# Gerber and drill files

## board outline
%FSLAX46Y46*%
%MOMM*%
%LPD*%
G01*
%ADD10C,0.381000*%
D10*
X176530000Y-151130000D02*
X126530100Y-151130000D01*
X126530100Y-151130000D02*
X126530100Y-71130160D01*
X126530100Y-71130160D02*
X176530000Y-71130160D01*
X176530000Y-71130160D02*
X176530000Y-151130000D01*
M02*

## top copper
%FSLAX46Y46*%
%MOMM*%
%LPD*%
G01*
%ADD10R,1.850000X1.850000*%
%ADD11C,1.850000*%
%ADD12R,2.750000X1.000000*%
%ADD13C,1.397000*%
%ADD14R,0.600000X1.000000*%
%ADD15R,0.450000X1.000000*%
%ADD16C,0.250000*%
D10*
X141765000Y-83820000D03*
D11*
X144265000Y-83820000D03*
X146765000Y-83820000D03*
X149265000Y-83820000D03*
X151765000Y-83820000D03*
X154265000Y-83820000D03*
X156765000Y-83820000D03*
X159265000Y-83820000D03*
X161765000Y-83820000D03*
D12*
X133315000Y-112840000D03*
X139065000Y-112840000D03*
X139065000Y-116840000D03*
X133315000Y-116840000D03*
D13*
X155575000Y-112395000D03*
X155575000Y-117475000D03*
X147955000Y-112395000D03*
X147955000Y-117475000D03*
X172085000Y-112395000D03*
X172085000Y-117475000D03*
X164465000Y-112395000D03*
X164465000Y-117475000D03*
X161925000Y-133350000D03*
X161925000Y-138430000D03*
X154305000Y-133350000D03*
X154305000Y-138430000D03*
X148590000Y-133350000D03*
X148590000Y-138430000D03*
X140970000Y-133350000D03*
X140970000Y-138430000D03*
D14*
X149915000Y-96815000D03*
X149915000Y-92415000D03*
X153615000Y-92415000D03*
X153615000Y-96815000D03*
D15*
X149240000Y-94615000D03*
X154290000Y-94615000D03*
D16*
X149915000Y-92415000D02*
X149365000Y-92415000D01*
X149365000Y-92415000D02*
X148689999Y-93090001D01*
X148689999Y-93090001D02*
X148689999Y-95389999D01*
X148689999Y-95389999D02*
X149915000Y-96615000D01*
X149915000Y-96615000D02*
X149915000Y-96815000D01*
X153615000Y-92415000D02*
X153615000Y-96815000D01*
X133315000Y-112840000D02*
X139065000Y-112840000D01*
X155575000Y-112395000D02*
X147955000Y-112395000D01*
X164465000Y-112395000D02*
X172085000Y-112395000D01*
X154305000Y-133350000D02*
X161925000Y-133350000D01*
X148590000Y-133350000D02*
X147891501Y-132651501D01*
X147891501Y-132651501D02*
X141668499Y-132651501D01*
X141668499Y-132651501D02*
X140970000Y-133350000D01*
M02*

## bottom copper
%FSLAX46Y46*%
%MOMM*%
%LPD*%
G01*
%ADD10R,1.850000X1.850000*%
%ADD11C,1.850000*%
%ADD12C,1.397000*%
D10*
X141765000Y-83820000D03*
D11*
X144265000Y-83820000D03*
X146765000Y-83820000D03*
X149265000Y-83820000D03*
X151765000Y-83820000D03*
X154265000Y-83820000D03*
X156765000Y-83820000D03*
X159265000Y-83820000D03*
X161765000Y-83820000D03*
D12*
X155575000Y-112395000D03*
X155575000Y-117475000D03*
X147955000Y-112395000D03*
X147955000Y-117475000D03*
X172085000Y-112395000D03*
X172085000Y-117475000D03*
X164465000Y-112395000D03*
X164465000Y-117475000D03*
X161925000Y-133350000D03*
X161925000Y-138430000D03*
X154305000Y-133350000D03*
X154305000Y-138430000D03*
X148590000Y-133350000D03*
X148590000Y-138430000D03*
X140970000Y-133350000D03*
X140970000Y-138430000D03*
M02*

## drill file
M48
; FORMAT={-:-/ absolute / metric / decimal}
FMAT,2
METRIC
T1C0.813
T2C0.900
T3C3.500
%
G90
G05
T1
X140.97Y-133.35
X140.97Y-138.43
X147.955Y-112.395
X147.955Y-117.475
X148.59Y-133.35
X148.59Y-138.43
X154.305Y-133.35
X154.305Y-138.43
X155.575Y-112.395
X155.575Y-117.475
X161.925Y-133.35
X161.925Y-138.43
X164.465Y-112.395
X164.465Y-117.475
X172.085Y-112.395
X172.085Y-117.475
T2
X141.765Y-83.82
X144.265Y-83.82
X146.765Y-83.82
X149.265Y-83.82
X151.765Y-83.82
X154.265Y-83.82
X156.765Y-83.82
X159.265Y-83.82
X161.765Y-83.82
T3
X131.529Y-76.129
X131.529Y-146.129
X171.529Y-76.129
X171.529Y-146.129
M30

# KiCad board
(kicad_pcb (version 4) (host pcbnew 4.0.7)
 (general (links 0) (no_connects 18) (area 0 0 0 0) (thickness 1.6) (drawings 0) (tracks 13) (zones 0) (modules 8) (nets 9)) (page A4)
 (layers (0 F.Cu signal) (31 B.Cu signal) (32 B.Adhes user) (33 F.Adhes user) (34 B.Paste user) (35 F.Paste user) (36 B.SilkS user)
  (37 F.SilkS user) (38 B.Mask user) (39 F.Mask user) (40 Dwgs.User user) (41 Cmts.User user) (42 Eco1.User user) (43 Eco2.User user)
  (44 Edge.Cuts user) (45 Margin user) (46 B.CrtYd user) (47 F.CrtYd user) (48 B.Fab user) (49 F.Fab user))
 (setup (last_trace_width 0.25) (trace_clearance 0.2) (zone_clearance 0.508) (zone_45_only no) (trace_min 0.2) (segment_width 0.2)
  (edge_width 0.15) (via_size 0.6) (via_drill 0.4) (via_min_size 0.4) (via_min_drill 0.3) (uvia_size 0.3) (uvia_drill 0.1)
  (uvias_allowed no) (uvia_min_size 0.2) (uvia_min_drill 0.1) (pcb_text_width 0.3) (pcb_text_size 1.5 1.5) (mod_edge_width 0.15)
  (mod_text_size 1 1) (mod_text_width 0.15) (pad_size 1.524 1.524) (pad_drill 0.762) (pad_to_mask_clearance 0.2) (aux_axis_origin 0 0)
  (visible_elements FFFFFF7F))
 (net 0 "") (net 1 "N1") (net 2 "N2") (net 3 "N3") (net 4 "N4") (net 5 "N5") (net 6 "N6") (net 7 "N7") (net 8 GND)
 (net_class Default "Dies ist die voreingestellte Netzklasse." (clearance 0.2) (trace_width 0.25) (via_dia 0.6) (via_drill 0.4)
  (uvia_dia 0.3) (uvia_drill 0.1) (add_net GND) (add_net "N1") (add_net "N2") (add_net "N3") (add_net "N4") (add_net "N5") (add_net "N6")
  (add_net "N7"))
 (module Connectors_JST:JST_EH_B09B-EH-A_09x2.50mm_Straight (layer B.Cu) (at 141.765 83.82)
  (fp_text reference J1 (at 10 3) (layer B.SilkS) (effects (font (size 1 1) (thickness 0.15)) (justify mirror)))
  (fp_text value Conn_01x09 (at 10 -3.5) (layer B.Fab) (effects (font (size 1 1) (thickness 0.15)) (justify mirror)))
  (pad 1 thru_hole rect (at 0 0) (size 1.85 1.85) (drill 0.9) (layers *.Cu *.Mask) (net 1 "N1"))
  (pad 2 thru_hole circle (at 2.5 0) (size 1.85 1.85) (drill 0.9) (layers *.Cu *.Mask) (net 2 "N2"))
  (pad 3 thru_hole circle (at 5 0) (size 1.85 1.85) (drill 0.9) (layers *.Cu *.Mask))
  (pad 4 thru_hole circle (at 7.5 0) (size 1.85 1.85) (drill 0.9) (layers *.Cu *.Mask) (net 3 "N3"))
  (pad 5 thru_hole circle (at 10 0) (size 1.85 1.85) (drill 0.9) (layers *.Cu *.Mask) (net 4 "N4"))
  (pad 6 thru_hole circle (at 12.5 0) (size 1.85 1.85) (drill 0.9) (layers *.Cu *.Mask) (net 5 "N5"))
  (pad 7 thru_hole circle (at 15 0) (size 1.85 1.85) (drill 0.9) (layers *.Cu *.Mask) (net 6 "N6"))
  (pad 8 thru_hole circle (at 17.5 0) (size 1.85 1.85) (drill 0.9) (layers *.Cu *.Mask) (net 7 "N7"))
  (pad 9 thru_hole circle (at 20 0) (size 1.85 1.85) (drill 0.9) (layers *.Cu *.Mask) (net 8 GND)))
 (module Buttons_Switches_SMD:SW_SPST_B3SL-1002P (layer F.Cu) (at 136.19 114.84)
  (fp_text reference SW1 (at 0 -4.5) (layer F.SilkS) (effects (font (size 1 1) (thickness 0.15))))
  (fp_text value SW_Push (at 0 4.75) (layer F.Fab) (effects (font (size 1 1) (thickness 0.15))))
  (pad 1 smd rect (at -2.875 -2) (size 2.75 1) (layers F.Cu F.Paste F.Mask) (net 3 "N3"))
  (pad 1 smd rect (at 2.875 -2) (size 2.75 1) (layers F.Cu F.Paste F.Mask) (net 3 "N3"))
  (pad 2 smd rect (at 2.875 2) (size 2.75 1) (layers F.Cu F.Paste F.Mask) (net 8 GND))
  (pad 2 smd rect (at -2.875 2) (size 2.75 1) (layers F.Cu F.Paste F.Mask) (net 8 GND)))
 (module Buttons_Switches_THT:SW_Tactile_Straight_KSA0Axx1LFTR (layer F.Cu) (at 147.955 112.395)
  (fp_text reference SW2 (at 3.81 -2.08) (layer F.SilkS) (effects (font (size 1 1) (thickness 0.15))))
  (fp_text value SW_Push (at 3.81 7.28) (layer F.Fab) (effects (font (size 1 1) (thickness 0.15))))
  (pad 1 thru_hole circle (at 7.62 0) (size 1.397 1.397) (drill 0.8128) (layers *.Cu *.Mask) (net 4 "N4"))
  (pad 2 thru_hole circle (at 7.62 5.08) (size 1.397 1.397) (drill 0.8128) (layers *.Cu *.Mask) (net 8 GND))
  (pad 1 thru_hole circle (at 0 0) (size 1.397 1.397) (drill 0.8128) (layers *.Cu *.Mask) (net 4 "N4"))
  (pad 2 thru_hole circle (at 0 5.08) (size 1.397 1.397) (drill 0.8128) (layers *.Cu *.Mask) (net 8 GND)))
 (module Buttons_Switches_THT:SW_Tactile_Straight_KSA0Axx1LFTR (layer F.Cu) (at 164.465 112.395)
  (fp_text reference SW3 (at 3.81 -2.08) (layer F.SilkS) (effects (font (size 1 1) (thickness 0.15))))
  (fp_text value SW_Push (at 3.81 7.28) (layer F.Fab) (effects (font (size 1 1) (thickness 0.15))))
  (pad 1 thru_hole circle (at 7.62 0) (size 1.397 1.397) (drill 0.8128) (layers *.Cu *.Mask) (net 5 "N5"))
  (pad 2 thru_hole circle (at 7.62 5.08) (size 1.397 1.397) (drill 0.8128) (layers *.Cu *.Mask) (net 8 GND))
  (pad 1 thru_hole circle (at 0 0) (size 1.397 1.397) (drill 0.8128) (layers *.Cu *.Mask) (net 5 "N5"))
  (pad 2 thru_hole circle (at 0 5.08) (size 1.397 1.397) (drill 0.8128) (layers *.Cu *.Mask) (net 8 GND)))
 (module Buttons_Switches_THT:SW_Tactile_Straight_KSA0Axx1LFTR (layer F.Cu) (at 154.305 133.35)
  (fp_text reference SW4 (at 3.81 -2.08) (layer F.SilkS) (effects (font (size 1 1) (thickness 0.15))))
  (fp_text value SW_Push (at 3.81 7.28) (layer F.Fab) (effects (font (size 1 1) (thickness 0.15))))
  (pad 1 thru_hole circle (at 7.62 0) (size 1.397 1.397) (drill 0.8128) (layers *.Cu *.Mask) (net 6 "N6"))
  (pad 2 thru_hole circle (at 7.62 5.08) (size 1.397 1.397) (drill 0.8128) (layers *.Cu *.Mask) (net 8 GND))
  (pad 1 thru_hole circle (at 0 0) (size 1.397 1.397) (drill 0.8128) (layers *.Cu *.Mask) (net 6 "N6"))
  (pad 2 thru_hole circle (at 0 5.08) (size 1.397 1.397) (drill 0.8128) (layers *.Cu *.Mask) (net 8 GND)))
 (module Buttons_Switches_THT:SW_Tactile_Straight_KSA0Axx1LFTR (layer F.Cu) (at 140.97 133.35)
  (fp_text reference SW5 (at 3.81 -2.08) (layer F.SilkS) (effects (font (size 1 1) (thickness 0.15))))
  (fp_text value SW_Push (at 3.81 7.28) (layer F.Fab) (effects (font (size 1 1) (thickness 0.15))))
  (pad 1 thru_hole circle (at 7.62 0) (size 1.397 1.397) (drill 0.8128) (layers *.Cu *.Mask) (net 7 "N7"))
  (pad 2 thru_hole circle (at 7.62 5.08) (size 1.397 1.397) (drill 0.8128) (layers *.Cu *.Mask) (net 8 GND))
  (pad 1 thru_hole circle (at 0 0) (size 1.397 1.397) (drill 0.8128) (layers *.Cu *.Mask) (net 7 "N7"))
  (pad 2 thru_hole circle (at 0 5.08) (size 1.397 1.397) (drill 0.8128) (layers *.Cu *.Mask) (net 8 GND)))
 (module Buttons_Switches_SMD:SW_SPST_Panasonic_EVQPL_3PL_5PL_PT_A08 (layer F.Cu) (at 151.765 94.615)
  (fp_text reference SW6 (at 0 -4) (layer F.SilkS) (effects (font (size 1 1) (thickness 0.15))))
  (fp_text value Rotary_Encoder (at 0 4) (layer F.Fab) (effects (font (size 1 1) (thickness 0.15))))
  (pad 1 smd rect (at -1.85 2.2) (size 0.6 1) (layers F.Cu F.Paste F.Mask) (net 1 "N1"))
  (pad 1 smd rect (at -1.85 -2.2) (size 0.6 1) (layers F.Cu F.Paste F.Mask) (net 1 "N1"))
  (pad 2 smd rect (at 1.85 -2.2) (size 0.6 1) (layers F.Cu F.Paste F.Mask) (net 2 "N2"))
  (pad 2 smd rect (at 1.85 2.2) (size 0.6 1) (layers F.Cu F.Paste F.Mask) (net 2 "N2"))
  (pad 0 smd rect (at -2.525 0) (size 0.45 1) (layers F.Cu F.Paste F.Mask))
  (pad 0 smd rect (at 2.525 0) (size 0.45 1) (layers F.Cu F.Paste F.Mask)))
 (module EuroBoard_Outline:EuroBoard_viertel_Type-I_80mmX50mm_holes (layer F.Cu) (at 176.53 151.13 90)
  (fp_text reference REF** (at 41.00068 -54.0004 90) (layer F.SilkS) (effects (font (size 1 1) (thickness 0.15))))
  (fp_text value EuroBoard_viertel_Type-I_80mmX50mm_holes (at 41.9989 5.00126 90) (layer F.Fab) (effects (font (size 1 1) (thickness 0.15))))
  (fp_line (start 0 0) (end 0 -49.9999) (layer Edge.Cuts) (width 0.381))
  (fp_line (start 0 -49.9999) (end 79.99984 -49.9999) (layer Edge.Cuts) (width 0.381))
  (fp_line (start 79.99984 -49.9999) (end 79.99984 0) (layer Edge.Cuts) (width 0.381))
  (fp_line (start 79.99984 0) (end 0 0) (layer Edge.Cuts) (width 0.381))
  (pad "" np_thru_hole circle (at 5.00126 -5.00126 90) (size 3.50012 3.50012) (drill 3.50012) (layers *.Cu *.Mask))
  (pad "" np_thru_hole circle (at 5.00126 -45.00118 90) (size 3.50012 3.50012) (drill 3.50012) (layers *.Cu *.Mask))
  (pad "" np_thru_hole circle (at 75.00112 -45.00118 90) (size 3.50012 3.50012) (drill 3.50012) (layers *.Cu *.Mask))
  (pad "" np_thru_hole circle (at 75.00112 -5.00126 90) (size 3.50012 3.50012) (drill 3.50012) (layers *.Cu *.Mask)))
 (segment (start 149.915 92.415) (end 149.365 92.415) (width 0.25) (layer F.Cu) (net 1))
 (segment (start 149.365 92.415) (end 148.689999 93.090001) (width 0.25) (layer F.Cu) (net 1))
 (segment (start 148.689999 93.090001) (end 148.689999 95.389999) (width 0.25) (layer F.Cu) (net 1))
 (segment (start 148.689999 95.389999) (end 149.915 96.615) (width 0.25) (layer F.Cu) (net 1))
 (segment (start 149.915 96.615) (end 149.915 96.815) (width 0.25) (layer F.Cu) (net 1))
 (segment (start 153.615 92.415) (end 153.615 96.815) (width 0.25) (layer F.Cu) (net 2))
 (segment (start 133.315 112.84) (end 139.065 112.84) (width 0.25) (layer F.Cu) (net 3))
 (segment (start 155.575 112.395) (end 147.955 112.395) (width 0.25) (layer F.Cu) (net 4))
 (segment (start 164.465 112.395) (end 172.085 112.395) (width 0.25) (layer F.Cu) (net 5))
 (segment (start 154.305 133.35) (end 161.925 133.35) (width 0.25) (layer F.Cu) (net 6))
 (segment (start 148.59 133.35) (end 147.891501 132.651501) (width 0.25) (layer F.Cu) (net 7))
 (segment (start 147.891501 132.651501) (end 141.668499 132.651501) (width 0.25) (layer F.Cu) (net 7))
 (segment (start 141.668499 132.651501) (end 140.97 133.35) (width 0.25) (layer F.Cu) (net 7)))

